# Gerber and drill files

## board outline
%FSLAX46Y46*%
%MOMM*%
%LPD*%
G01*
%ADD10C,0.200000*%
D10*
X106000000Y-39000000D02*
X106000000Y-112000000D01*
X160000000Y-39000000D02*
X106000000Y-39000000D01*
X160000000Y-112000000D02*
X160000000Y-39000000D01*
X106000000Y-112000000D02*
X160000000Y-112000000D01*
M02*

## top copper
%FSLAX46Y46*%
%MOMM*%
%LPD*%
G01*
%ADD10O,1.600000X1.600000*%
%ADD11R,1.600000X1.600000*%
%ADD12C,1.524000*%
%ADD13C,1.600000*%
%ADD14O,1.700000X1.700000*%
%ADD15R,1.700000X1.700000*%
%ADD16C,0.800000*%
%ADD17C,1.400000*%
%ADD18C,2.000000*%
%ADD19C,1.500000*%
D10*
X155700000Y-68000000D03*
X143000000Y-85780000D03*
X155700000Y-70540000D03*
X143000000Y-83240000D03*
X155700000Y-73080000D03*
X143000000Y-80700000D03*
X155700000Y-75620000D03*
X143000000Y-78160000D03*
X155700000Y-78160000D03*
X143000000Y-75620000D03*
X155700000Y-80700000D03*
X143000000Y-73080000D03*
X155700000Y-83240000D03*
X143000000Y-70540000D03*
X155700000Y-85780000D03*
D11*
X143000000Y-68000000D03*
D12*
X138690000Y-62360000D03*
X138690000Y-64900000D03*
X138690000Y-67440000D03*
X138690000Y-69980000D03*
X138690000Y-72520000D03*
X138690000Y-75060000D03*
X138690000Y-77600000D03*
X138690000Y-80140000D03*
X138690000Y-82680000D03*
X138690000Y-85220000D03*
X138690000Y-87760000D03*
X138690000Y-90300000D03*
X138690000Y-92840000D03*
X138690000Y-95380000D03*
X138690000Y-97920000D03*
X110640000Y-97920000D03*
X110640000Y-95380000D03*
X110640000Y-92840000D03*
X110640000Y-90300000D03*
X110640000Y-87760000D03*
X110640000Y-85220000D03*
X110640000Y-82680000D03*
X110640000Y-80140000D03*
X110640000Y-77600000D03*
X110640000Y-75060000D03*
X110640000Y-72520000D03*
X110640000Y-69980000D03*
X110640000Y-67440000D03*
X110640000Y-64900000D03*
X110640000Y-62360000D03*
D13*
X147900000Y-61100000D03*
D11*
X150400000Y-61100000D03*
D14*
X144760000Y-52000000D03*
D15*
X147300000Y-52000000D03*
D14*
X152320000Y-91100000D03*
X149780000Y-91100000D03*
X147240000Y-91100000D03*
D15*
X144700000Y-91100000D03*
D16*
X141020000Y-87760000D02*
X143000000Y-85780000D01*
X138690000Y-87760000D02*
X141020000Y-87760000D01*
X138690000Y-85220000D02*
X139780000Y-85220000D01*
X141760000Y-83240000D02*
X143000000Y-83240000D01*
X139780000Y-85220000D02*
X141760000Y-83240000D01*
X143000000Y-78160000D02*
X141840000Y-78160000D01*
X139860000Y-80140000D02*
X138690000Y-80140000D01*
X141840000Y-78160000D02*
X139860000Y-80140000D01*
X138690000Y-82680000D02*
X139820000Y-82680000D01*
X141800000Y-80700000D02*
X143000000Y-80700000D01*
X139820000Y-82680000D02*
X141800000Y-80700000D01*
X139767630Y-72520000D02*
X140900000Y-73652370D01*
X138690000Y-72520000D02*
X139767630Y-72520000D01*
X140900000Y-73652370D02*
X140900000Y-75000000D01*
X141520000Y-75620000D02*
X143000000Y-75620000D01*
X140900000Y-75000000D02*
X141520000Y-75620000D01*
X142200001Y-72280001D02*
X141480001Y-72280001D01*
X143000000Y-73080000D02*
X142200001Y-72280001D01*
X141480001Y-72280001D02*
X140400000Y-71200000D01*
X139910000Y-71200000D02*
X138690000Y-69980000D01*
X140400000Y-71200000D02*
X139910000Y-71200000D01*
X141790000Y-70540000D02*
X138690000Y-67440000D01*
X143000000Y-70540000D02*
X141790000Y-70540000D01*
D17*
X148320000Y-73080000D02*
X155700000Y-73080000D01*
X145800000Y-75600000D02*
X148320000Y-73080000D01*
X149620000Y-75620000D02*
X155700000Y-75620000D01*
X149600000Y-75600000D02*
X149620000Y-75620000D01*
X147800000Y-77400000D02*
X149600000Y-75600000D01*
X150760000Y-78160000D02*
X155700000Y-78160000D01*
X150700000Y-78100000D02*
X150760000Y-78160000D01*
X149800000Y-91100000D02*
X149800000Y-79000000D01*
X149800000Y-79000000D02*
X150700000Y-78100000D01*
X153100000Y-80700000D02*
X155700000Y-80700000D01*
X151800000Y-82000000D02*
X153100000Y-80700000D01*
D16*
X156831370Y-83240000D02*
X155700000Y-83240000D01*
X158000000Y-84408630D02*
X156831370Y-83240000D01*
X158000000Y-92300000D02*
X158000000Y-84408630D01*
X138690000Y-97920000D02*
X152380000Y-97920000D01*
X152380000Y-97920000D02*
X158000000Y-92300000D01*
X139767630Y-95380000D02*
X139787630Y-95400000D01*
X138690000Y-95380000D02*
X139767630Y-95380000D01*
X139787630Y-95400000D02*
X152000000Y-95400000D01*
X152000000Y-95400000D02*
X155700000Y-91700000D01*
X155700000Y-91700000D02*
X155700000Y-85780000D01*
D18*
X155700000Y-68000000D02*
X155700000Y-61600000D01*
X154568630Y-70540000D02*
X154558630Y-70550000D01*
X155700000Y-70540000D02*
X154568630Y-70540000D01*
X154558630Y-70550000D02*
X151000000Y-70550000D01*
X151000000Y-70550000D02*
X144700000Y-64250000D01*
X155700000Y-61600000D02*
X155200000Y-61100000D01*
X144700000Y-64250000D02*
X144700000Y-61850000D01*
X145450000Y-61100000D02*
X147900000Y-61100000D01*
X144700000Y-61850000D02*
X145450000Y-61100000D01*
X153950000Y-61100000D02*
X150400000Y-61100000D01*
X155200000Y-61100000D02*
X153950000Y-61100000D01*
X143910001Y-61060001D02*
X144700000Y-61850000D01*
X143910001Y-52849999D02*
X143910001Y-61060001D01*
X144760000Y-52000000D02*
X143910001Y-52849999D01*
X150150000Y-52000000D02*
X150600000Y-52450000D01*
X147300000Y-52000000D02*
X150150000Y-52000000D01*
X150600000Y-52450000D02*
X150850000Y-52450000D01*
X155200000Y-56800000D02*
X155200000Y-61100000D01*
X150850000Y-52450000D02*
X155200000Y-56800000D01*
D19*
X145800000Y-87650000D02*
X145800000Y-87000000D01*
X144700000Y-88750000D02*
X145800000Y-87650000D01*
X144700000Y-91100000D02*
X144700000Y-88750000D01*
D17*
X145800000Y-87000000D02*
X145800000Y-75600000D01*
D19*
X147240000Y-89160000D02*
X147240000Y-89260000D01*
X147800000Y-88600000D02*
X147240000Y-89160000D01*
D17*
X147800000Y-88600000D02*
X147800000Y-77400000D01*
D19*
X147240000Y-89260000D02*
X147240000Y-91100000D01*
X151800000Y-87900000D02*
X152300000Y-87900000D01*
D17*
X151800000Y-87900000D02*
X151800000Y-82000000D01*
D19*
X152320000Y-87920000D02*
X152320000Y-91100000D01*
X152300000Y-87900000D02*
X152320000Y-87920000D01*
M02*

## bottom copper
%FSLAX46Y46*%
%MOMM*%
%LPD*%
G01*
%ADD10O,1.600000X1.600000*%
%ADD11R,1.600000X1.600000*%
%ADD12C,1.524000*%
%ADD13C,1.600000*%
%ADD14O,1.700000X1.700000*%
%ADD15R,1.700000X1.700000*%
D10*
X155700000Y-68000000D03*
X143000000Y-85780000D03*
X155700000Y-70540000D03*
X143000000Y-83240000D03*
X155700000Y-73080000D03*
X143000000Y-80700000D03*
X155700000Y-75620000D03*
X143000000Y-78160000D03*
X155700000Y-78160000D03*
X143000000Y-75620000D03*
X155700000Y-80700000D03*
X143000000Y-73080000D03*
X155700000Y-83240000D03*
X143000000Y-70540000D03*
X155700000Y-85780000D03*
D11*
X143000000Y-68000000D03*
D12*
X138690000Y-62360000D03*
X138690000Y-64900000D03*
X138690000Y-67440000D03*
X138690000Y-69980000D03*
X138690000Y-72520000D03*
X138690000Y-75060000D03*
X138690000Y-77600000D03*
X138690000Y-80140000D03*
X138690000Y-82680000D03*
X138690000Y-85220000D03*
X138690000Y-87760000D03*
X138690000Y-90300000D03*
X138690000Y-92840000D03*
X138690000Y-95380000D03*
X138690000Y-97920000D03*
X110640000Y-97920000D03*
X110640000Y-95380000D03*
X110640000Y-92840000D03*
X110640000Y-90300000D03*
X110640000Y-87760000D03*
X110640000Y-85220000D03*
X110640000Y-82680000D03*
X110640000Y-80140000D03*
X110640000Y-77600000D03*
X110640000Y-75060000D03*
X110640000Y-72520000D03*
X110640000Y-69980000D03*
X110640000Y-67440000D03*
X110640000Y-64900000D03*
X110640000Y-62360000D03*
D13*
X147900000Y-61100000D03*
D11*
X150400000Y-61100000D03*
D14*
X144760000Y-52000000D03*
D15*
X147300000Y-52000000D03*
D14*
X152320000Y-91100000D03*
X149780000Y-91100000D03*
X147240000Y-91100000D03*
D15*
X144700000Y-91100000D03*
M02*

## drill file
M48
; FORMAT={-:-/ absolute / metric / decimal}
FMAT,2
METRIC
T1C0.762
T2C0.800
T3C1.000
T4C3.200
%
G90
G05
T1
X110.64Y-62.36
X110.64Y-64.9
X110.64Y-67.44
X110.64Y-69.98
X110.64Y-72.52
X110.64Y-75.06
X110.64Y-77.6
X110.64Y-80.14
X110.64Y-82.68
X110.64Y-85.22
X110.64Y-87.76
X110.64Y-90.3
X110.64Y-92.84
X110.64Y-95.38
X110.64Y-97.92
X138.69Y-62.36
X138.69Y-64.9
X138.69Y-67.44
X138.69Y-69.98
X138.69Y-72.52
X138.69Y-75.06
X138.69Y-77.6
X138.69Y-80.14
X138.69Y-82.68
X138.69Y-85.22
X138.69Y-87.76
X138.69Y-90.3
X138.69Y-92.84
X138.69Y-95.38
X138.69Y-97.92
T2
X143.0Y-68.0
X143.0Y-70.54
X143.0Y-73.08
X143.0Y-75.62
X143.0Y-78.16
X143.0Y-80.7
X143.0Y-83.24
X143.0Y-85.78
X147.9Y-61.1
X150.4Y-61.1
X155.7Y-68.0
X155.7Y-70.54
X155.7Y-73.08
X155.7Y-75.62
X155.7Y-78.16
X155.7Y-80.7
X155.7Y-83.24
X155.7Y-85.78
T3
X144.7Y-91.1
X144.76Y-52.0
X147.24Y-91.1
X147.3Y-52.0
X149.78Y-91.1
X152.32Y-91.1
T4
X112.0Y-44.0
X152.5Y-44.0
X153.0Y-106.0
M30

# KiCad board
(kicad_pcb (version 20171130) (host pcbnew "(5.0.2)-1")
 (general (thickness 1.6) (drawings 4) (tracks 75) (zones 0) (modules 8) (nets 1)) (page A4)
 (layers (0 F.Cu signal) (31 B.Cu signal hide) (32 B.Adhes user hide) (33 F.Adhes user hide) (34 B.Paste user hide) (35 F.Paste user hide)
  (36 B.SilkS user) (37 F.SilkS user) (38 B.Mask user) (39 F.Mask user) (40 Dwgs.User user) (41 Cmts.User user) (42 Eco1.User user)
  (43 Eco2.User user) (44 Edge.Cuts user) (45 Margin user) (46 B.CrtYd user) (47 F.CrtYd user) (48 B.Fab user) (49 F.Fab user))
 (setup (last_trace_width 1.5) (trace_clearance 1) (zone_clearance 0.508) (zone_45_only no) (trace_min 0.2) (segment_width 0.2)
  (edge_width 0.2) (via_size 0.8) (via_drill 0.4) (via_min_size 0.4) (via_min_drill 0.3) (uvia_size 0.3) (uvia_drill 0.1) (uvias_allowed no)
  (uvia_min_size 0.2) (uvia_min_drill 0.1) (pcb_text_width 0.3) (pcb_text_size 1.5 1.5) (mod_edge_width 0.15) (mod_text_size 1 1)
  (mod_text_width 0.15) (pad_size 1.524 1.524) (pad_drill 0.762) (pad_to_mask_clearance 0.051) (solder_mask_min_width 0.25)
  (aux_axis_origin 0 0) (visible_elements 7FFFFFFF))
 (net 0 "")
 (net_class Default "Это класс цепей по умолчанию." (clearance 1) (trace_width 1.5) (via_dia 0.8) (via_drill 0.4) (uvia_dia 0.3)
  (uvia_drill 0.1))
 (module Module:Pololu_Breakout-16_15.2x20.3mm (layer F.Cu) (at 143 68)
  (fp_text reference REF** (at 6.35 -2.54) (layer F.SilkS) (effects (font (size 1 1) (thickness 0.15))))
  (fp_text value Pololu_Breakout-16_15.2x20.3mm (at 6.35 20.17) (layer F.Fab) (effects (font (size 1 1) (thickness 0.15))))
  (pad 16 thru_hole oval (at 12.7 0) (size 1.6 1.6) (drill 0.8) (layers *.Cu *.Mask))
  (pad 8 thru_hole oval (at 0 17.78) (size 1.6 1.6) (drill 0.8) (layers *.Cu *.Mask))
  (pad 15 thru_hole oval (at 12.7 2.54) (size 1.6 1.6) (drill 0.8) (layers *.Cu *.Mask))
  (pad 7 thru_hole oval (at 0 15.24) (size 1.6 1.6) (drill 0.8) (layers *.Cu *.Mask))
  (pad 14 thru_hole oval (at 12.7 5.08) (size 1.6 1.6) (drill 0.8) (layers *.Cu *.Mask))
  (pad 6 thru_hole oval (at 0 12.7) (size 1.6 1.6) (drill 0.8) (layers *.Cu *.Mask))
  (pad 13 thru_hole oval (at 12.7 7.62) (size 1.6 1.6) (drill 0.8) (layers *.Cu *.Mask))
  (pad 5 thru_hole oval (at 0 10.16) (size 1.6 1.6) (drill 0.8) (layers *.Cu *.Mask))
  (pad 12 thru_hole oval (at 12.7 10.16) (size 1.6 1.6) (drill 0.8) (layers *.Cu *.Mask))
  (pad 4 thru_hole oval (at 0 7.62) (size 1.6 1.6) (drill 0.8) (layers *.Cu *.Mask))
  (pad 11 thru_hole oval (at 12.7 12.7) (size 1.6 1.6) (drill 0.8) (layers *.Cu *.Mask))
  (pad 3 thru_hole oval (at 0 5.08) (size 1.6 1.6) (drill 0.8) (layers *.Cu *.Mask))
  (pad 10 thru_hole oval (at 12.7 15.24) (size 1.6 1.6) (drill 0.8) (layers *.Cu *.Mask))
  (pad 2 thru_hole oval (at 0 2.54) (size 1.6 1.6) (drill 0.8) (layers *.Cu *.Mask))
  (pad 9 thru_hole oval (at 12.7 17.78) (size 1.6 1.6) (drill 0.8) (layers *.Cu *.Mask))
  (pad 1 thru_hole rect (at 0 0) (size 1.6 1.6) (drill 0.8) (layers *.Cu *.Mask)))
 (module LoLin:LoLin (layer F.Cu) (at 108.9 52.2)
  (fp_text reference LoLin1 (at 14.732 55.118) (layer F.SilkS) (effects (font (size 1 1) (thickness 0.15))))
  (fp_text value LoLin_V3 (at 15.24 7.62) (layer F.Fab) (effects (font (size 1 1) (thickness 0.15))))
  (pad 30 thru_hole circle (at 29.79 10.16) (size 1.524 1.524) (drill 0.762) (layers *.Cu *.Mask F.SilkS))
  (pad 29 thru_hole circle (at 29.79 12.7) (size 1.524 1.524) (drill 0.762) (layers *.Cu *.Mask F.SilkS))
  (pad 28 thru_hole circle (at 29.79 15.24) (size 1.524 1.524) (drill 0.762) (layers *.Cu *.Mask F.SilkS))
  (pad 27 thru_hole circle (at 29.79 17.78) (size 1.524 1.524) (drill 0.762) (layers *.Cu *.Mask F.SilkS))
  (pad 26 thru_hole circle (at 29.79 20.32) (size 1.524 1.524) (drill 0.762) (layers *.Cu *.Mask F.SilkS))
  (pad 25 thru_hole circle (at 29.79 22.86) (size 1.524 1.524) (drill 0.762) (layers *.Cu *.Mask F.SilkS))
  (pad 24 thru_hole circle (at 29.79 25.4) (size 1.524 1.524) (drill 0.762) (layers *.Cu *.Mask F.SilkS))
  (pad 23 thru_hole circle (at 29.79 27.94) (size 1.524 1.524) (drill 0.762) (layers *.Cu *.Mask F.SilkS))
  (pad 22 thru_hole circle (at 29.79 30.48) (size 1.524 1.524) (drill 0.762) (layers *.Cu *.Mask F.SilkS))
  (pad 21 thru_hole circle (at 29.79 33.02) (size 1.524 1.524) (drill 0.762) (layers *.Cu *.Mask F.SilkS))
  (pad 20 thru_hole circle (at 29.79 35.56) (size 1.524 1.524) (drill 0.762) (layers *.Cu *.Mask F.SilkS))
  (pad 19 thru_hole circle (at 29.79 38.1) (size 1.524 1.524) (drill 0.762) (layers *.Cu *.Mask F.SilkS))
  (pad 18 thru_hole circle (at 29.79 40.64) (size 1.524 1.524) (drill 0.762) (layers *.Cu *.Mask F.SilkS))
  (pad 17 thru_hole circle (at 29.79 43.18) (size 1.524 1.524) (drill 0.762) (layers *.Cu *.Mask F.SilkS))
  (pad 16 thru_hole circle (at 29.79 45.72) (size 1.524 1.524) (drill 0.762) (layers *.Cu *.Mask F.SilkS))
  (pad 15 thru_hole circle (at 1.74 45.72) (size 1.524 1.524) (drill 0.762) (layers *.Cu *.Mask F.SilkS))
  (pad 14 thru_hole circle (at 1.74 43.18) (size 1.524 1.524) (drill 0.762) (layers *.Cu *.Mask F.SilkS))
  (pad 13 thru_hole circle (at 1.74 40.64) (size 1.524 1.524) (drill 0.762) (layers *.Cu *.Mask F.SilkS))
  (pad 12 thru_hole circle (at 1.74 38.1) (size 1.524 1.524) (drill 0.762) (layers *.Cu *.Mask F.SilkS))
  (pad 11 thru_hole circle (at 1.74 35.56) (size 1.524 1.524) (drill 0.762) (layers *.Cu *.Mask F.SilkS))
  (pad 10 thru_hole circle (at 1.74 33.02) (size 1.524 1.524) (drill 0.762) (layers *.Cu *.Mask F.SilkS))
  (pad 9 thru_hole circle (at 1.74 30.48) (size 1.524 1.524) (drill 0.762) (layers *.Cu *.Mask F.SilkS))
  (pad 8 thru_hole circle (at 1.74 27.94) (size 1.524 1.524) (drill 0.762) (layers *.Cu *.Mask F.SilkS))
  (pad 7 thru_hole circle (at 1.74 25.4) (size 1.524 1.524) (drill 0.762) (layers *.Cu *.Mask F.SilkS))
  (pad 6 thru_hole circle (at 1.74 22.86) (size 1.524 1.524) (drill 0.762) (layers *.Cu *.Mask F.SilkS))
  (pad 5 thru_hole circle (at 1.74 20.32) (size 1.524 1.524) (drill 0.762) (layers *.Cu *.Mask F.SilkS))
  (pad 4 thru_hole circle (at 1.74 17.78) (size 1.524 1.524) (drill 0.762) (layers *.Cu *.Mask F.SilkS))
  (pad 3 thru_hole circle (at 1.74 15.24) (size 1.524 1.524) (drill 0.762) (layers *.Cu *.Mask F.SilkS))
  (pad 2 thru_hole circle (at 1.74 12.7) (size 1.524 1.524) (drill 0.762) (layers *.Cu *.Mask F.SilkS))
  (pad 1 thru_hole circle (at 1.74 10.16) (size 1.524 1.524) (drill 0.762) (layers *.Cu *.Mask F.SilkS)))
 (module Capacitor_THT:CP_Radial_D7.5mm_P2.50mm (layer F.Cu) (at 150.4 61.1 180)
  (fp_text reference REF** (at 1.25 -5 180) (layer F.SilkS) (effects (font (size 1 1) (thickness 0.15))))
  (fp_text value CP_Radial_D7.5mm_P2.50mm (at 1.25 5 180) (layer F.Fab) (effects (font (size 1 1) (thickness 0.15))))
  (pad 2 thru_hole circle (at 2.5 0 180) (size 1.6 1.6) (drill 0.8) (layers *.Cu *.Mask))
  (pad 1 thru_hole rect (at 0 0 180) (size 1.6 1.6) (drill 0.8) (layers *.Cu *.Mask)))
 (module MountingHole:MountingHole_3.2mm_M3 (layer F.Cu) (at 112 44)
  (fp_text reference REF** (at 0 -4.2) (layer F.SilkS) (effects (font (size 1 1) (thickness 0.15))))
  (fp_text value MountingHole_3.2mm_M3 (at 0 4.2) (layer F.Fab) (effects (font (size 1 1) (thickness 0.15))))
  (pad 1 np_thru_hole circle (at 0 0) (size 3.2 3.2) (drill 3.2) (layers *.Cu *.Mask)))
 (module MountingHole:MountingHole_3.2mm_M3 (layer F.Cu) (at 153 106)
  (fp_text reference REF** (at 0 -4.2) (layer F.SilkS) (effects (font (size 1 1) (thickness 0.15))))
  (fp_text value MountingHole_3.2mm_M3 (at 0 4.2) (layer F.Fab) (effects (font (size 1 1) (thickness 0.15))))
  (pad 1 np_thru_hole circle (at 0 0) (size 3.2 3.2) (drill 3.2) (layers *.Cu *.Mask)))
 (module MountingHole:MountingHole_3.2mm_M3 (layer F.Cu) (at 152.5 44)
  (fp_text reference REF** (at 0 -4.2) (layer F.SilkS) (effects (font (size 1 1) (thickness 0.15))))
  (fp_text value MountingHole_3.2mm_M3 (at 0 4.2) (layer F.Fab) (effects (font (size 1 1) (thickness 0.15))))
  (pad 1 np_thru_hole circle (at 0 0) (size 3.2 3.2) (drill 3.2) (layers *.Cu *.Mask)))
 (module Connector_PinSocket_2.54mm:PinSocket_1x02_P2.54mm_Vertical (layer F.Cu) (at 147.3 52 270)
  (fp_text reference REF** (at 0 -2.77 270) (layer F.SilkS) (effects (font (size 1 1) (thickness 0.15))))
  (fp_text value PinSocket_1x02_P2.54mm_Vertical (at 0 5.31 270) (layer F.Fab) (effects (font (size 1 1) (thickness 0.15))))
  (pad 2 thru_hole oval (at 0 2.54 270) (size 1.7 1.7) (drill 1) (layers *.Cu *.Mask))
  (pad 1 thru_hole rect (at 0 0 270) (size 1.7 1.7) (drill 1) (layers *.Cu *.Mask)))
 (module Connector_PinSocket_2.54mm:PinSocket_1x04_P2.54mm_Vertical (layer F.Cu) (at 144.7 91.1 90)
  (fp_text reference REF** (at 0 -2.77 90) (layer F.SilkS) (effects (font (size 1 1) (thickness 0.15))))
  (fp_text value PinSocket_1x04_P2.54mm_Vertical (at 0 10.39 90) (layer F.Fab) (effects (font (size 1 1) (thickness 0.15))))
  (pad 4 thru_hole oval (at 0 7.62 90) (size 1.7 1.7) (drill 1) (layers *.Cu *.Mask))
  (pad 3 thru_hole oval (at 0 5.08 90) (size 1.7 1.7) (drill 1) (layers *.Cu *.Mask))
  (pad 2 thru_hole oval (at 0 2.54 90) (size 1.7 1.7) (drill 1) (layers *.Cu *.Mask))
  (pad 1 thru_hole rect (at 0 0 90) (size 1.7 1.7) (drill 1) (layers *.Cu *.Mask)))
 (gr_line (start 106 39) (end 106 112) (layer Edge.Cuts) (width 0.2))
 (gr_line (start 160 39) (end 106 39) (layer Edge.Cuts) (width 0.2))
 (gr_line (start 160 112) (end 160 39) (layer Edge.Cuts) (width 0.2))
 (gr_line (start 106 112) (end 160 112) (layer Edge.Cuts) (width 0.2))
 (segment (start 141.02 87.76) (end 143 85.78) (width 0.8) (layer F.Cu) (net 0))
 (segment (start 138.69 87.76) (end 141.02 87.76) (width 0.8) (layer F.Cu) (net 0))
 (segment (start 138.69 85.22) (end 139.78 85.22) (width 0.8) (layer F.Cu) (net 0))
 (segment (start 141.76 83.24) (end 143 83.24) (width 0.8) (layer F.Cu) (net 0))
 (segment (start 139.78 85.22) (end 141.76 83.24) (width 0.8) (layer F.Cu) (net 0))
 (segment (start 143 78.16) (end 141.84 78.16) (width 0.8) (layer F.Cu) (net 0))
 (segment (start 139.86 80.14) (end 138.69 80.14) (width 0.8) (layer F.Cu) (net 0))
 (segment (start 141.84 78.16) (end 139.86 80.14) (width 0.8) (layer F.Cu) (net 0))
 (segment (start 138.69 82.68) (end 139.82 82.68) (width 0.8) (layer F.Cu) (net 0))
 (segment (start 141.8 80.7) (end 143 80.7) (width 0.8) (layer F.Cu) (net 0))
 (segment (start 139.82 82.68) (end 141.8 80.7) (width 0.8) (layer F.Cu) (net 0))
 (segment (start 139.76763 72.52) (end 140.9 73.65237) (width 0.8) (layer F.Cu) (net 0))
 (segment (start 138.69 72.52) (end 139.76763 72.52) (width 0.8) (layer F.Cu) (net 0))
 (segment (start 140.9 73.65237) (end 140.9 75) (width 0.8) (layer F.Cu) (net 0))
 (segment (start 141.52 75.62) (end 143 75.62) (width 0.8) (layer F.Cu) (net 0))
 (segment (start 140.9 75) (end 141.52 75.62) (width 0.8) (layer F.Cu) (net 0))
 (segment (start 142.200001 72.280001) (end 141.480001 72.280001) (width 0.8) (layer F.Cu) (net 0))
 (segment (start 143 73.08) (end 142.200001 72.280001) (width 0.8) (layer F.Cu) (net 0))
 (segment (start 141.480001 72.280001) (end 140.4 71.2) (width 0.8) (layer F.Cu) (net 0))
 (segment (start 139.91 71.2) (end 138.69 69.98) (width 0.8) (layer F.Cu) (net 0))
 (segment (start 140.4 71.2) (end 139.91 71.2) (width 0.8) (layer F.Cu) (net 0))
 (segment (start 141.79 70.54) (end 138.69 67.44) (width 0.8) (layer F.Cu) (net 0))
 (segment (start 143 70.54) (end 141.79 70.54) (width 0.8) (layer F.Cu) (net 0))
 (segment (start 148.32 73.08) (end 155.7 73.08) (width 1.4) (layer F.Cu) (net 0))
 (segment (start 145.8 75.6) (end 148.32 73.08) (width 1.4) (layer F.Cu) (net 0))
 (segment (start 149.62 75.62) (end 155.7 75.62) (width 1.4) (layer F.Cu) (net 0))
 (segment (start 149.6 75.6) (end 149.62 75.62) (width 1.4) (layer F.Cu) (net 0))
 (segment (start 147.8 77.4) (end 149.6 75.6) (width 1.4) (layer F.Cu) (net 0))
 (segment (start 150.76 78.16) (end 155.7 78.16) (width 1.4) (layer F.Cu) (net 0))
 (segment (start 150.7 78.1) (end 150.76 78.16) (width 1.4) (layer F.Cu) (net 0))
 (segment (start 149.8 91.1) (end 149.8 79) (width 1.4) (layer F.Cu) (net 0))
 (segment (start 149.8 79) (end 150.7 78.1) (width 1.4) (layer F.Cu) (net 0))
 (segment (start 153.1 80.7) (end 155.7 80.7) (width 1.4) (layer F.Cu) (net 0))
 (segment (start 151.8 82) (end 153.1 80.7) (width 1.4) (layer F.Cu) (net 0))
 (segment (start 156.83137 83.24) (end 155.7 83.24) (width 0.8) (layer F.Cu) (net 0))
 (segment (start 158 84.40863) (end 156.83137 83.24) (width 0.8) (layer F.Cu) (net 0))
 (segment (start 158 92.3) (end 158 84.40863) (width 0.8) (layer F.Cu) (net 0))
 (segment (start 138.69 97.92) (end 152.38 97.92) (width 0.8) (layer F.Cu) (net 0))
 (segment (start 152.38 97.92) (end 158 92.3) (width 0.8) (layer F.Cu) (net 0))
 (segment (start 139.76763 95.38) (end 139.78763 95.4) (width 0.8) (layer F.Cu) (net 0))
 (segment (start 138.69 95.38) (end 139.76763 95.38) (width 0.8) (layer F.Cu) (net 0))
 (segment (start 139.78763 95.4) (end 152 95.4) (width 0.8) (layer F.Cu) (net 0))
 (segment (start 152 95.4) (end 155.7 91.7) (width 0.8) (layer F.Cu) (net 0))
 (segment (start 155.7 91.7) (end 155.7 85.78) (width 0.8) (layer F.Cu) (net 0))
 (segment (start 155.7 68) (end 155.7 61.6) (width 2) (layer F.Cu) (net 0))
 (segment (start 154.56863 70.54) (end 154.55863 70.55) (width 2) (layer F.Cu) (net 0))
 (segment (start 155.7 70.54) (end 154.56863 70.54) (width 2) (layer F.Cu) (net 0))
 (segment (start 154.55863 70.55) (end 151 70.55) (width 2) (layer F.Cu) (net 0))
 (segment (start 151 70.55) (end 144.7 64.25) (width 2) (layer F.Cu) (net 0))
 (segment (start 155.7 61.6) (end 155.2 61.1) (width 2) (layer F.Cu) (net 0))
 (segment (start 144.7 64.25) (end 144.7 61.85) (width 2) (layer F.Cu) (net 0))
 (segment (start 145.45 61.1) (end 147.9 61.1) (width 2) (layer F.Cu) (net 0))
 (segment (start 144.7 61.85) (end 145.45 61.1) (width 2) (layer F.Cu) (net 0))
 (segment (start 153.95 61.1) (end 150.4 61.1) (width 2) (layer F.Cu) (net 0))
 (segment (start 155.2 61.1) (end 153.95 61.1) (width 2) (layer F.Cu) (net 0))
 (segment (start 143.910001 61.060001) (end 144.7 61.85) (width 2) (layer F.Cu) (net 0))
 (segment (start 143.910001 52.849999) (end 143.910001 61.060001) (width 2) (layer F.Cu) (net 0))
 (segment (start 144.76 52) (end 143.910001 52.849999) (width 2) (layer F.Cu) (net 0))
 (segment (start 150.15 52) (end 150.6 52.45) (width 2) (layer F.Cu) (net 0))
 (segment (start 147.3 52) (end 150.15 52) (width 2) (layer F.Cu) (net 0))
 (segment (start 150.6 52.45) (end 150.85 52.45) (width 2) (layer F.Cu) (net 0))
 (segment (start 155.2 56.8) (end 155.2 61.1) (width 2) (layer F.Cu) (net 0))
 (segment (start 150.85 52.45) (end 155.2 56.8) (width 2) (layer F.Cu) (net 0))
 (segment (start 145.8 87.65) (end 145.8 87) (width 1.5) (layer F.Cu) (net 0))
 (segment (start 144.7 88.75) (end 145.8 87.65) (width 1.5) (layer F.Cu) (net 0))
 (segment (start 144.7 91.1) (end 144.7 88.75) (width 1.5) (layer F.Cu) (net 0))
 (segment (start 145.8 87) (end 145.8 75.6) (width 1.4) (layer F.Cu) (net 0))
 (segment (start 147.24 89.16) (end 147.24 89.26) (width 1.5) (layer F.Cu) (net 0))
 (segment (start 147.8 88.6) (end 147.24 89.16) (width 1.5) (layer F.Cu) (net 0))
 (segment (start 147.8 88.6) (end 147.8 77.4) (width 1.4) (layer F.Cu) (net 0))
 (segment (start 147.24 89.26) (end 147.24 91.1) (width 1.5) (layer F.Cu) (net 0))
 (segment (start 151.8 87.9) (end 152.3 87.9) (width 1.5) (layer F.Cu) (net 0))
 (segment (start 151.8 87.9) (end 151.8 82) (width 1.4) (layer F.Cu) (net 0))
 (segment (start 152.32 87.92) (end 152.32 91.1) (width 1.5) (layer F.Cu) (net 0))
 (segment (start 152.3 87.9) (end 152.32 87.92) (width 1.5) (layer F.Cu) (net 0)))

